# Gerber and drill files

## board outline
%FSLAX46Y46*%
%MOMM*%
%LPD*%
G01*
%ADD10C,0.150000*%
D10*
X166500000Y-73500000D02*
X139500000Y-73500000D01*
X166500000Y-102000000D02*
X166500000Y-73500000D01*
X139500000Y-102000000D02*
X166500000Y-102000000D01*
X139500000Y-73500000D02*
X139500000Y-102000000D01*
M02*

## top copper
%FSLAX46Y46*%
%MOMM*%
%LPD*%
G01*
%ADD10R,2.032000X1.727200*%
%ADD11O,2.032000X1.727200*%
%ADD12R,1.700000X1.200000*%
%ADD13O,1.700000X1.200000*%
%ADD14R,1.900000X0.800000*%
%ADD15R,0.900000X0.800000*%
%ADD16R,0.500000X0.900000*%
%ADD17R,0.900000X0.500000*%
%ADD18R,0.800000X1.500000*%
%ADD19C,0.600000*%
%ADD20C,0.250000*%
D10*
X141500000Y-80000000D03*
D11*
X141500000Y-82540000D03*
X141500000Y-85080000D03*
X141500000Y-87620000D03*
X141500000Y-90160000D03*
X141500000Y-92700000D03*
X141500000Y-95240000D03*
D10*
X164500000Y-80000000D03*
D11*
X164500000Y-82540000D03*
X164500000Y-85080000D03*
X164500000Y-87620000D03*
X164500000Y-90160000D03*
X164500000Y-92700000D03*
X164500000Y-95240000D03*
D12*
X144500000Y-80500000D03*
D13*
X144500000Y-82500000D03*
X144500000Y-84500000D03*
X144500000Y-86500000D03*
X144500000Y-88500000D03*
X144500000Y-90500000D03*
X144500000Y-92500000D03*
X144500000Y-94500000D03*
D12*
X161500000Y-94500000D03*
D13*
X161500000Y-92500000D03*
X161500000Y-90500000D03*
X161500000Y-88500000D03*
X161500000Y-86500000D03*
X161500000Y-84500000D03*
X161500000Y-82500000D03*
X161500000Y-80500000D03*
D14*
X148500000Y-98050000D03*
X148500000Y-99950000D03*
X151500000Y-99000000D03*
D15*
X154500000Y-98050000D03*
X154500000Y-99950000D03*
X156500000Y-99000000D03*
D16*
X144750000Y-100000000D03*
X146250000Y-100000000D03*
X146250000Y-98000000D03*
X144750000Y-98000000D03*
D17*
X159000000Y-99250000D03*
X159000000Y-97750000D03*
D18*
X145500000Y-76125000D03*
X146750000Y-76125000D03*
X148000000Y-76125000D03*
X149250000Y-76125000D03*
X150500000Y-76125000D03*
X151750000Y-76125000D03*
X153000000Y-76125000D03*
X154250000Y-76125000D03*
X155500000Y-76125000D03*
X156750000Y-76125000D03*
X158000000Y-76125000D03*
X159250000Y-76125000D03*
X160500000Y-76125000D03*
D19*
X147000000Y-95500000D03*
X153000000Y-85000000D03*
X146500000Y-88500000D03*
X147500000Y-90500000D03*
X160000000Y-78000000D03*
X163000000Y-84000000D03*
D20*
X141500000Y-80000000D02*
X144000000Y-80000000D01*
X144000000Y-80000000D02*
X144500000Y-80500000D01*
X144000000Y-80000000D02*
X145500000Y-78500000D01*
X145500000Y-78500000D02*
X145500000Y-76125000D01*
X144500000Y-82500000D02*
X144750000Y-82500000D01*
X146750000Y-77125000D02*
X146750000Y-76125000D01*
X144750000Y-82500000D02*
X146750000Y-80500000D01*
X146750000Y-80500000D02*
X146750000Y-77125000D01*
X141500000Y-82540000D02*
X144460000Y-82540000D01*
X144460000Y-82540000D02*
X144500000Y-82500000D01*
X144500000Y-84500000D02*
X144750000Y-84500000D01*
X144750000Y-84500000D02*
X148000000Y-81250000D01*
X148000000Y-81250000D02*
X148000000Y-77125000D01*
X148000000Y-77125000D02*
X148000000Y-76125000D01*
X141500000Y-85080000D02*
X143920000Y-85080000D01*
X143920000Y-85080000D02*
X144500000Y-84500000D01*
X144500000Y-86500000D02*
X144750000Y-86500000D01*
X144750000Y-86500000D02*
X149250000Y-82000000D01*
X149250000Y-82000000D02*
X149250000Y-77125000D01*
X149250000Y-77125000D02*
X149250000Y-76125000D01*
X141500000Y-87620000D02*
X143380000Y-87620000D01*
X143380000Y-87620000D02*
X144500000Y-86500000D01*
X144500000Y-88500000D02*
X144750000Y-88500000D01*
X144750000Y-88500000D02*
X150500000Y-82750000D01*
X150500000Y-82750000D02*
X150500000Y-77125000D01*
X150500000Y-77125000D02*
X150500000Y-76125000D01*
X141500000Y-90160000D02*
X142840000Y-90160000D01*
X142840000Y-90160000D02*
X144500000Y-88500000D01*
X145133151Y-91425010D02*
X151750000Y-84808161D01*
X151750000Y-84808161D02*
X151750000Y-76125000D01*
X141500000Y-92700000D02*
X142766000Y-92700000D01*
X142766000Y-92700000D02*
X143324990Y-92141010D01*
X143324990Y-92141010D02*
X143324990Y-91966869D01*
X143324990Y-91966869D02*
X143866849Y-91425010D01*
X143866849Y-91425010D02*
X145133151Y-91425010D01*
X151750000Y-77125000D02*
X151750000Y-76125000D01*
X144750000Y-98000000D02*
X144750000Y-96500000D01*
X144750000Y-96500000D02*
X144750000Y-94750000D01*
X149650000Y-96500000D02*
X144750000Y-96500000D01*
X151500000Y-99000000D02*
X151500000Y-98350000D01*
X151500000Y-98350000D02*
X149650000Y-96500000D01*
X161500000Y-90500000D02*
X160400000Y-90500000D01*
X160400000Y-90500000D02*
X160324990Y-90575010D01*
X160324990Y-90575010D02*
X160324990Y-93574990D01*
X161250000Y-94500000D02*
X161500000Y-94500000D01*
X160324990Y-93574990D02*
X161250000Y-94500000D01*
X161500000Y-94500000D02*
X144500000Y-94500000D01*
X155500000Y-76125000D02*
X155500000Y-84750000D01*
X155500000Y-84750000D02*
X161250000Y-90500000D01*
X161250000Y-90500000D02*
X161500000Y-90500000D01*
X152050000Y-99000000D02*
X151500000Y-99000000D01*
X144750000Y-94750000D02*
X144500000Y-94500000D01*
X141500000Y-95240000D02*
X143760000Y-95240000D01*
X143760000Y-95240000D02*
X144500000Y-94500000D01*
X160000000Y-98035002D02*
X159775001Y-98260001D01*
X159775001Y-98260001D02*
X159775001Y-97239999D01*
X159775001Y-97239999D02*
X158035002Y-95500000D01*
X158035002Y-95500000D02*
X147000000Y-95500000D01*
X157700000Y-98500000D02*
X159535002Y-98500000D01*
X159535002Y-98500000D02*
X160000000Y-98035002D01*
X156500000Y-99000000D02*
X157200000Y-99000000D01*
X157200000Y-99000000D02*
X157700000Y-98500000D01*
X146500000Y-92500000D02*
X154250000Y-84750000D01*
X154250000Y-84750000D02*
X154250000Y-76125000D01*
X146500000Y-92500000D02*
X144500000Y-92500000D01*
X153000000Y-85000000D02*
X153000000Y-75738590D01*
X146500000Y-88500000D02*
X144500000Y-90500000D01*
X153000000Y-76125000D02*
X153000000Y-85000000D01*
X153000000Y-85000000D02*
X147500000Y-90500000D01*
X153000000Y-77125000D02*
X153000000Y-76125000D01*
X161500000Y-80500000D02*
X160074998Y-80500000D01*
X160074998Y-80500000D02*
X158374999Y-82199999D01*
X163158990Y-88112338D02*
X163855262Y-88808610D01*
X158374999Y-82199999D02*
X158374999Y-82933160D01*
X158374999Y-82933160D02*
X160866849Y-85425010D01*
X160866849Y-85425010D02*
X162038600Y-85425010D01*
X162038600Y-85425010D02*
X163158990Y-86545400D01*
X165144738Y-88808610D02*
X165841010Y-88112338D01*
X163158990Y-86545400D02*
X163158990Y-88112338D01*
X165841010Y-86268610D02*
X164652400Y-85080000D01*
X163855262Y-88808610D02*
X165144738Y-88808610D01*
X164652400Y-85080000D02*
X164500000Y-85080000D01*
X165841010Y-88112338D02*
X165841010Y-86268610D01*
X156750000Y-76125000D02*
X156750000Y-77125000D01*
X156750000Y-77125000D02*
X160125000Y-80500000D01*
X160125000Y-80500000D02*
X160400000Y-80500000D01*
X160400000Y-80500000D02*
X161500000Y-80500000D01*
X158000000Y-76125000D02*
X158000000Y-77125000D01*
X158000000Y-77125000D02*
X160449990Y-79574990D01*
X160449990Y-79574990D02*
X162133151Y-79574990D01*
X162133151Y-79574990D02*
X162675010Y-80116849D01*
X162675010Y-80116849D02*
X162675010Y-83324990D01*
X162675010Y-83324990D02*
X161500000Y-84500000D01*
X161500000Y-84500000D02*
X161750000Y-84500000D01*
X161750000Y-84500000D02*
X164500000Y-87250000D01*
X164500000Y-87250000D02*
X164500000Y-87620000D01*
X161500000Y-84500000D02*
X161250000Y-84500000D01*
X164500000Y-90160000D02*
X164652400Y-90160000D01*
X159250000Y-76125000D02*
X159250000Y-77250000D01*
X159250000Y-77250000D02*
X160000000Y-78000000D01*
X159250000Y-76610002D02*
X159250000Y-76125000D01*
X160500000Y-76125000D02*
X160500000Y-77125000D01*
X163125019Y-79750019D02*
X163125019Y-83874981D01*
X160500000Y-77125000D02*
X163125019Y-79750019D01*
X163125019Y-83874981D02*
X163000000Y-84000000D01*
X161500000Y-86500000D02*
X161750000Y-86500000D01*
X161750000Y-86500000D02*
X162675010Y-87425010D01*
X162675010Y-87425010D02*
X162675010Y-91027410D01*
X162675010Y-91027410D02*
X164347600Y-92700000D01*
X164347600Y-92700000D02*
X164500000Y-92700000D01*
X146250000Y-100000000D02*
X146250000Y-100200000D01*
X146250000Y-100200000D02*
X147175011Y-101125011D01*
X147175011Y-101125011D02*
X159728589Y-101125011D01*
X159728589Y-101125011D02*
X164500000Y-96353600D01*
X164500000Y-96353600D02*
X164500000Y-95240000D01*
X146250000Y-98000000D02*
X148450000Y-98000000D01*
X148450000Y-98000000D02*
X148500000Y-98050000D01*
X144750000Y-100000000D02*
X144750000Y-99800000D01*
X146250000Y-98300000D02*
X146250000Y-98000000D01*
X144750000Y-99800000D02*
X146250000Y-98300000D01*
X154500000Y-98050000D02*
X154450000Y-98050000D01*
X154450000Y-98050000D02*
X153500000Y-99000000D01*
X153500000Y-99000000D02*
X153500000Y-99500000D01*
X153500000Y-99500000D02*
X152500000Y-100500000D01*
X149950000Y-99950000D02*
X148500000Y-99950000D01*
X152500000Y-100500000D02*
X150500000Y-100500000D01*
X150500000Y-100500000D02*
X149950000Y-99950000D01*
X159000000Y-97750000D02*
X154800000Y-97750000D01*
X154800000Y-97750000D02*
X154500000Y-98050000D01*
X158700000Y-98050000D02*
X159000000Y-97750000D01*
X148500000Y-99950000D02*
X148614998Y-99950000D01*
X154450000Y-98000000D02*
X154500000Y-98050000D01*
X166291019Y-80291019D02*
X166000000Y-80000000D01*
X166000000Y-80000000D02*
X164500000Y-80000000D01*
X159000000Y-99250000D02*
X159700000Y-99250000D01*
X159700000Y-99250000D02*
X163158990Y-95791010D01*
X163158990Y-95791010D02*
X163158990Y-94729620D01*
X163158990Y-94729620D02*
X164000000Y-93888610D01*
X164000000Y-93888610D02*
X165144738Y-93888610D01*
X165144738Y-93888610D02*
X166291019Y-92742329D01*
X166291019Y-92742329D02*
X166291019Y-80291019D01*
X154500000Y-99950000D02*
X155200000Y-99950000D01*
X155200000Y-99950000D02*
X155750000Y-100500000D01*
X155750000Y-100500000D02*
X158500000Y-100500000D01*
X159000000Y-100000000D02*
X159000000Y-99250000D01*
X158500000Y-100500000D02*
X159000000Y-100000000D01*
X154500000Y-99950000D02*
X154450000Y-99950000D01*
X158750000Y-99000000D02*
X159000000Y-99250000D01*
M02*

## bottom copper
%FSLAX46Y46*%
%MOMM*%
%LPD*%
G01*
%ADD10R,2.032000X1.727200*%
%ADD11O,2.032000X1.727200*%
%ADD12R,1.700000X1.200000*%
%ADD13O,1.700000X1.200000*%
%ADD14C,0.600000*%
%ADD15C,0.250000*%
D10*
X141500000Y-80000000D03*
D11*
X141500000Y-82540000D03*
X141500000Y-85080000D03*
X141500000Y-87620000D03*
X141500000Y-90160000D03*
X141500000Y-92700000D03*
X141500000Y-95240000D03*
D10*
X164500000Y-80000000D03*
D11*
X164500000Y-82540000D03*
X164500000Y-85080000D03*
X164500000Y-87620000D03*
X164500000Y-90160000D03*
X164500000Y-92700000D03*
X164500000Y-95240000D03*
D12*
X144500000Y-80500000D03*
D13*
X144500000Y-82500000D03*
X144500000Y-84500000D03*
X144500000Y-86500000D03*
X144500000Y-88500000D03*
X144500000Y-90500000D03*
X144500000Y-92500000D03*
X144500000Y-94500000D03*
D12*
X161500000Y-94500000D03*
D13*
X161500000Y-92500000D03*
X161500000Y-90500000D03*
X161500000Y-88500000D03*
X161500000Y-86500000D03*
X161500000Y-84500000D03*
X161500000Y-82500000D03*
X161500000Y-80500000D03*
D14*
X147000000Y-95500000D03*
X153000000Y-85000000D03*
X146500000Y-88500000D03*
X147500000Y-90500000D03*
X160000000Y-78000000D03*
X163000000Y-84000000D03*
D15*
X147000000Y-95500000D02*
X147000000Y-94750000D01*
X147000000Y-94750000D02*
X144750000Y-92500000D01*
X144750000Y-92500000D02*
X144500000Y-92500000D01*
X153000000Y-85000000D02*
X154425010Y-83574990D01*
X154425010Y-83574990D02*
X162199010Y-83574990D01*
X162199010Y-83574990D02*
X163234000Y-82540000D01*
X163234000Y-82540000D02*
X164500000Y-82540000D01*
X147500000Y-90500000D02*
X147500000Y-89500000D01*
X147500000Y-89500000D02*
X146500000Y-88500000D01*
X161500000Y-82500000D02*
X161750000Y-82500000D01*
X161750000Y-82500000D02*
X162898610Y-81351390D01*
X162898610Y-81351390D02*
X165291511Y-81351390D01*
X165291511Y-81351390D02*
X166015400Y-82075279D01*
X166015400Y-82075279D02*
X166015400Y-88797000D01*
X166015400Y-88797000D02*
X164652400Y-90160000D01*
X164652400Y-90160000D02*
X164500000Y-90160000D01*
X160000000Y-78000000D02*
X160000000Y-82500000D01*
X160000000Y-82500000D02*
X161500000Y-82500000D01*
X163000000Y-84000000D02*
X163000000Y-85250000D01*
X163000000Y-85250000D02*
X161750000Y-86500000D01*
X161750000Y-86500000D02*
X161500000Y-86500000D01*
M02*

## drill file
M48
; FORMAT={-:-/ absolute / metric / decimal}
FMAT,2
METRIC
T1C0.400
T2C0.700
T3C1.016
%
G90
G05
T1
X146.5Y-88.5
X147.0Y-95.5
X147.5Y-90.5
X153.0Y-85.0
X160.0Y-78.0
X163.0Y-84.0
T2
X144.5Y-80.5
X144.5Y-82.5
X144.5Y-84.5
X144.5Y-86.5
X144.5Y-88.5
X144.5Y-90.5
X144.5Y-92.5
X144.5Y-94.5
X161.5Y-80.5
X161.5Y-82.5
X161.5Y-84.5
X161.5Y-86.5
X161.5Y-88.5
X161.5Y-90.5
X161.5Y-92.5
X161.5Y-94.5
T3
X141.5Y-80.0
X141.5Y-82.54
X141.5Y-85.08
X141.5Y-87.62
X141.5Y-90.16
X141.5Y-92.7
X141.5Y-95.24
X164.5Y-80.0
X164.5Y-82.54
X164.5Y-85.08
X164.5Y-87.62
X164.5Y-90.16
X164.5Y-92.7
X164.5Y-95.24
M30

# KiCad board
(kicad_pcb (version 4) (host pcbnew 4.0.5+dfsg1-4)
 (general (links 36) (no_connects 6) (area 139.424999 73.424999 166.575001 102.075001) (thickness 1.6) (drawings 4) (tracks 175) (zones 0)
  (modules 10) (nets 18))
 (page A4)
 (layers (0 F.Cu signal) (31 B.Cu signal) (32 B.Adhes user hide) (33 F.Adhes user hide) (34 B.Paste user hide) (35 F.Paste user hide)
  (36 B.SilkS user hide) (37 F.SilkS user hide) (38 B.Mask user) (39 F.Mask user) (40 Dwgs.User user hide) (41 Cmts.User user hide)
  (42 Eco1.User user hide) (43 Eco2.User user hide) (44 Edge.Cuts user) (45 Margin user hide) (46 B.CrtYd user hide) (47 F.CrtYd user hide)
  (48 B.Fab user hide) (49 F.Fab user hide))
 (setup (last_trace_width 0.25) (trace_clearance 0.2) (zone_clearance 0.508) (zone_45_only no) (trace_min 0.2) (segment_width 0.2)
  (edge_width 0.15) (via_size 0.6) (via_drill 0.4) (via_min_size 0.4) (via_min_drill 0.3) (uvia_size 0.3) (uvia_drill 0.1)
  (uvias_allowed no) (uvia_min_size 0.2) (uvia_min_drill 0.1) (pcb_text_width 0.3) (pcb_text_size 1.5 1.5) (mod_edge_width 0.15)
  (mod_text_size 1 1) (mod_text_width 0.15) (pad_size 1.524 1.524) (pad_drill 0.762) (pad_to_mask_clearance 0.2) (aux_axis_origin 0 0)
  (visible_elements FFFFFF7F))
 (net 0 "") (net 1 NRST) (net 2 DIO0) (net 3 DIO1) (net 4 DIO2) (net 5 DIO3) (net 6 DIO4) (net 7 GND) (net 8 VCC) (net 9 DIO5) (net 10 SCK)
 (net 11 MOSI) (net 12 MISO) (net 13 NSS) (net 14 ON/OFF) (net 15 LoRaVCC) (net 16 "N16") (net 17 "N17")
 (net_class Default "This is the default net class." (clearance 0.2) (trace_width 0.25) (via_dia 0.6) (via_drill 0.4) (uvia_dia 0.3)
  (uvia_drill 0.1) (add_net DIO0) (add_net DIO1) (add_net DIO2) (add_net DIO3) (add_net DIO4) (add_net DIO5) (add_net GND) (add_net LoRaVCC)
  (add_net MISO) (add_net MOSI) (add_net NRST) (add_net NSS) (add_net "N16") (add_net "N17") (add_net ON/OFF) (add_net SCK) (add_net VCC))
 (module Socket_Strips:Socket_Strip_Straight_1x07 (layer F.Cu) (at 141.5 80 270)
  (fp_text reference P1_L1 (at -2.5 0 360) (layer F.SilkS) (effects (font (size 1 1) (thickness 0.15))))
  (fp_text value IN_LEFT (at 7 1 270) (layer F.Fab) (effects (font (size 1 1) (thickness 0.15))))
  (pad 1 thru_hole rect (at 0 0 270) (size 1.7272 2.032) (drill 1.016) (layers *.Cu *.Mask) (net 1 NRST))
  (pad 2 thru_hole oval (at 2.54 0 270) (size 1.7272 2.032) (drill 1.016) (layers *.Cu *.Mask) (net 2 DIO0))
  (pad 3 thru_hole oval (at 5.08 0 270) (size 1.7272 2.032) (drill 1.016) (layers *.Cu *.Mask) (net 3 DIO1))
  (pad 4 thru_hole oval (at 7.62 0 270) (size 1.7272 2.032) (drill 1.016) (layers *.Cu *.Mask) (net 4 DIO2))
  (pad 5 thru_hole oval (at 10.16 0 270) (size 1.7272 2.032) (drill 1.016) (layers *.Cu *.Mask) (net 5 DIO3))
  (pad 6 thru_hole oval (at 12.7 0 270) (size 1.7272 2.032) (drill 1.016) (layers *.Cu *.Mask) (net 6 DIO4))
  (pad 7 thru_hole oval (at 15.24 0 270) (size 1.7272 2.032) (drill 1.016) (layers *.Cu *.Mask) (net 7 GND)))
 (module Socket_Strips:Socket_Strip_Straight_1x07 (layer F.Cu) (at 164.5 80 270)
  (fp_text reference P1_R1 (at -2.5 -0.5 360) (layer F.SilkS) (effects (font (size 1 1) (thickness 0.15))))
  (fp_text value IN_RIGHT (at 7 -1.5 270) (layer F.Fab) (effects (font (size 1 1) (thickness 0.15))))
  (pad 1 thru_hole rect (at 0 0 270) (size 1.7272 2.032) (drill 1.016) (layers *.Cu *.Mask) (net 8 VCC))
  (pad 2 thru_hole oval (at 2.54 0 270) (size 1.7272 2.032) (drill 1.016) (layers *.Cu *.Mask) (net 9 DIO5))
  (pad 3 thru_hole oval (at 5.08 0 270) (size 1.7272 2.032) (drill 1.016) (layers *.Cu *.Mask) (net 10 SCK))
  (pad 4 thru_hole oval (at 7.62 0 270) (size 1.7272 2.032) (drill 1.016) (layers *.Cu *.Mask) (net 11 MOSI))
  (pad 5 thru_hole oval (at 10.16 0 270) (size 1.7272 2.032) (drill 1.016) (layers *.Cu *.Mask) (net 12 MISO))
  (pad 6 thru_hole oval (at 12.7 0 270) (size 1.7272 2.032) (drill 1.016) (layers *.Cu *.Mask) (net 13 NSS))
  (pad 7 thru_hole oval (at 15.24 0 270) (size 1.7272 2.032) (drill 1.016) (layers *.Cu *.Mask) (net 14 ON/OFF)))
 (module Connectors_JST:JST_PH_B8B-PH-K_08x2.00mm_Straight (layer F.Cu) (at 144.5 80.5 270)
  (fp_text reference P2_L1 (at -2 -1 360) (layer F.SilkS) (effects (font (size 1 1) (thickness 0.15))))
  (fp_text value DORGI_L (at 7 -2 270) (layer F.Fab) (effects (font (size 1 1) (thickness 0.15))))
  (pad 1 thru_hole rect (at 0 0 270) (size 1.2 1.7) (drill 0.7) (layers *.Cu *.Mask) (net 1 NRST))
  (pad 2 thru_hole oval (at 2 0 270) (size 1.2 1.7) (drill 0.7) (layers *.Cu *.Mask) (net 2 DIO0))
  (pad 3 thru_hole oval (at 4 0 270) (size 1.2 1.7) (drill 0.7) (layers *.Cu *.Mask) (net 3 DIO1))
  (pad 4 thru_hole oval (at 6 0 270) (size 1.2 1.7) (drill 0.7) (layers *.Cu *.Mask) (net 4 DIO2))
  (pad 5 thru_hole oval (at 8 0 270) (size 1.2 1.7) (drill 0.7) (layers *.Cu *.Mask) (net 5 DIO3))
  (pad 6 thru_hole oval (at 10 0 270) (size 1.2 1.7) (drill 0.7) (layers *.Cu *.Mask) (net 9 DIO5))
  (pad 7 thru_hole oval (at 12 0 270) (size 1.2 1.7) (drill 0.7) (layers *.Cu *.Mask) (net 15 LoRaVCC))
  (pad 8 thru_hole oval (at 14 0 270) (size 1.2 1.7) (drill 0.7) (layers *.Cu *.Mask) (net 7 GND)))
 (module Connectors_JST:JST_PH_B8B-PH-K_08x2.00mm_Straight (layer F.Cu) (at 161.5 94.5 90)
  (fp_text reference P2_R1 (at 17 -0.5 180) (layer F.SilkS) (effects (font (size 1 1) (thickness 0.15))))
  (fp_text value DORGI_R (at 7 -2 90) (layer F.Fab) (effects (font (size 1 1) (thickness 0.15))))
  (pad 1 thru_hole rect (at 0 0 90) (size 1.2 1.7) (drill 0.7) (layers *.Cu *.Mask) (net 7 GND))
  (pad 2 thru_hole oval (at 2 0 90) (size 1.2 1.7) (drill 0.7) (layers *.Cu *.Mask))
  (pad 3 thru_hole oval (at 4 0 90) (size 1.2 1.7) (drill 0.7) (layers *.Cu *.Mask) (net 7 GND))
  (pad 4 thru_hole oval (at 6 0 90) (size 1.2 1.7) (drill 0.7) (layers *.Cu *.Mask))
  (pad 5 thru_hole oval (at 8 0 90) (size 1.2 1.7) (drill 0.7) (layers *.Cu *.Mask) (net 13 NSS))
  (pad 6 thru_hole oval (at 10 0 90) (size 1.2 1.7) (drill 0.7) (layers *.Cu *.Mask) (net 11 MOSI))
  (pad 7 thru_hole oval (at 12 0 90) (size 1.2 1.7) (drill 0.7) (layers *.Cu *.Mask) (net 12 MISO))
  (pad 8 thru_hole oval (at 14 0 90) (size 1.2 1.7) (drill 0.7) (layers *.Cu *.Mask) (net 10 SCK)))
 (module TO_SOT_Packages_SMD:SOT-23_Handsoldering (layer F.Cu) (at 150 99)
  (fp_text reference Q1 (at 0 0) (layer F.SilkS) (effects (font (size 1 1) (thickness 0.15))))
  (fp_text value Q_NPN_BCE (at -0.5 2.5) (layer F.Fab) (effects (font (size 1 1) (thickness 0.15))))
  (pad 1 smd rect (at -1.5 -0.95) (size 1.9 0.8) (layers F.Cu F.Paste F.Mask) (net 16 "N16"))
  (pad 2 smd rect (at -1.5 0.95) (size 1.9 0.8) (layers F.Cu F.Paste F.Mask) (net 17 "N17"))
  (pad 3 smd rect (at 1.5 0) (size 1.9 0.8) (layers F.Cu F.Paste F.Mask) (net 7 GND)))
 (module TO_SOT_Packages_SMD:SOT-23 (layer F.Cu) (at 155.5 99)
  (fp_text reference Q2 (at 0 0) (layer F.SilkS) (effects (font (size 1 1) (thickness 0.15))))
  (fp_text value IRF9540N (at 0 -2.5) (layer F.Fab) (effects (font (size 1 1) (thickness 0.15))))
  (pad 1 smd rect (at -1 -0.95) (size 0.9 0.8) (layers F.Cu F.Paste F.Mask) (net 17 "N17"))
  (pad 2 smd rect (at -1 0.95) (size 0.9 0.8) (layers F.Cu F.Paste F.Mask) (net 8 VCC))
  (pad 3 smd rect (at 1 0) (size 0.9 0.8) (layers F.Cu F.Paste F.Mask) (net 15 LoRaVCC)))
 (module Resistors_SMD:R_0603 (layer F.Cu) (at 145.5 100)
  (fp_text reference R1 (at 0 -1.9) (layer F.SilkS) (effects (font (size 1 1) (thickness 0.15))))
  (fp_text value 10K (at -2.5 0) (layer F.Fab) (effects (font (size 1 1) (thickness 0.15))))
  (pad 1 smd rect (at -0.75 0) (size 0.5 0.9) (layers F.Cu F.Paste F.Mask) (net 16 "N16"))
  (pad 2 smd rect (at 0.75 0) (size 0.5 0.9) (layers F.Cu F.Paste F.Mask) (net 14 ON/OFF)))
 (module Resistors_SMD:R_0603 (layer F.Cu) (at 145.5 98 180)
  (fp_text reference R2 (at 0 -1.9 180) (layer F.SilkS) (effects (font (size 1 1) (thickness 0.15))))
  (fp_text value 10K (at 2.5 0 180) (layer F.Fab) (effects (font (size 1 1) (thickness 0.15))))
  (pad 1 smd rect (at -0.75 0 180) (size 0.5 0.9) (layers F.Cu F.Paste F.Mask) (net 16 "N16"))
  (pad 2 smd rect (at 0.75 0 180) (size 0.5 0.9) (layers F.Cu F.Paste F.Mask) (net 7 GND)))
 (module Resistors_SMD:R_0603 (layer F.Cu) (at 159 98.5 90)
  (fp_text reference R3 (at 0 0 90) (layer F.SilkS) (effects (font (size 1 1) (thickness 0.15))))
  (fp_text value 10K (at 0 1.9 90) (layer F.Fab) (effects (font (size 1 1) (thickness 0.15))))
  (pad 1 smd rect (at -0.75 0 90) (size 0.5 0.9) (layers F.Cu F.Paste F.Mask) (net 8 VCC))
  (pad 2 smd rect (at 0.75 0 90) (size 0.5 0.9) (layers F.Cu F.Paste F.Mask) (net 17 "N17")))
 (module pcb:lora (layer F.Cu) (at 153 77.5)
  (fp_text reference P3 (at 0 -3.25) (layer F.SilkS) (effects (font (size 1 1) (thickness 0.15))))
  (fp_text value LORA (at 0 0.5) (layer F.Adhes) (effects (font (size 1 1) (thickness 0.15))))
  (pad 1 smd rect (at -7.5 -1.375) (size 0.8 1.5) (layers F.Cu F.Paste F.Mask) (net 1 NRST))
  (pad 2 smd rect (at -6.25 -1.375) (size 0.8 1.5) (layers F.Cu F.Paste F.Mask) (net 2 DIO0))
  (pad 3 smd rect (at -5 -1.375) (size 0.8 1.5) (layers F.Cu F.Paste F.Mask) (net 3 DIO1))
  (pad 4 smd rect (at -3.75 -1.375) (size 0.8 1.5) (layers F.Cu F.Paste F.Mask) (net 4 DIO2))
  (pad 5 smd rect (at -2.5 -1.375) (size 0.8 1.5) (layers F.Cu F.Paste F.Mask) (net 5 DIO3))
  (pad 6 smd rect (at -1.25 -1.375) (size 0.8 1.5) (layers F.Cu F.Paste F.Mask) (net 6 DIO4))
  (pad 7 smd rect (at 0 -1.375) (size 0.8 1.5) (layers F.Cu F.Paste F.Mask) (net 9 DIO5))
  (pad 8 smd rect (at 1.25 -1.375) (size 0.8 1.5) (layers F.Cu F.Paste F.Mask) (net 15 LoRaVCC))
  (pad 9 smd rect (at 2.5 -1.375) (size 0.8 1.5) (layers F.Cu F.Paste F.Mask) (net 7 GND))
  (pad 10 smd rect (at 3.75 -1.375) (size 0.8 1.5) (layers F.Cu F.Paste F.Mask) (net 10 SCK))
  (pad 11 smd rect (at 5 -1.375) (size 0.8 1.5) (layers F.Cu F.Paste F.Mask) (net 11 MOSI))
  (pad 12 smd rect (at 6.25 -1.375) (size 0.8 1.5) (layers F.Cu F.Paste F.Mask) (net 12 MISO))
  (pad 13 smd rect (at 7.5 -1.375) (size 0.8 1.5) (layers F.Cu F.Paste F.Mask) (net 13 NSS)))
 (gr_line (start 166.5 73.5) (end 139.5 73.5) (layer Edge.Cuts) (width 0.15))
 (gr_line (start 166.5 102) (end 166.5 73.5) (layer Edge.Cuts) (width 0.15))
 (gr_line (start 139.5 102) (end 166.5 102) (layer Edge.Cuts) (width 0.15))
 (gr_line (start 139.5 73.5) (end 139.5 102) (layer Edge.Cuts) (width 0.15))
 (segment (start 141.5 80) (end 144 80) (width 0.25) (layer F.Cu) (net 1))
 (segment (start 144 80) (end 144.5 80.5) (width 0.25) (layer F.Cu) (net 1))
 (segment (start 144 80) (end 145.5 78.5) (width 0.25) (layer F.Cu) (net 1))
 (segment (start 145.5 78.5) (end 145.5 76.125) (width 0.25) (layer F.Cu) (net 1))
 (segment (start 144.5 82.5) (end 144.75 82.5) (width 0.25) (layer F.Cu) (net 2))
 (segment (start 146.75 77.125) (end 146.75 76.125) (width 0.25) (layer F.Cu) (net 2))
 (segment (start 144.75 82.5) (end 146.75 80.5) (width 0.25) (layer F.Cu) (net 2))
 (segment (start 146.75 80.5) (end 146.75 77.125) (width 0.25) (layer F.Cu) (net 2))
 (segment (start 141.5 82.54) (end 144.46 82.54) (width 0.25) (layer F.Cu) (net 2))
 (segment (start 144.46 82.54) (end 144.5 82.5) (width 0.25) (layer F.Cu) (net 2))
 (segment (start 144.5 84.5) (end 144.75 84.5) (width 0.25) (layer F.Cu) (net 3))
 (segment (start 144.75 84.5) (end 148 81.25) (width 0.25) (layer F.Cu) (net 3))
 (segment (start 148 81.25) (end 148 77.125) (width 0.25) (layer F.Cu) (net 3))
 (segment (start 148 77.125) (end 148 76.125) (width 0.25) (layer F.Cu) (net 3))
 (segment (start 141.5 85.08) (end 143.92 85.08) (width 0.25) (layer F.Cu) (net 3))
 (segment (start 143.92 85.08) (end 144.5 84.5) (width 0.25) (layer F.Cu) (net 3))
 (segment (start 144.5 86.5) (end 144.75 86.5) (width 0.25) (layer F.Cu) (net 4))
 (segment (start 144.75 86.5) (end 149.25 82) (width 0.25) (layer F.Cu) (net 4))
 (segment (start 149.25 82) (end 149.25 77.125) (width 0.25) (layer F.Cu) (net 4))
 (segment (start 149.25 77.125) (end 149.25 76.125) (width 0.25) (layer F.Cu) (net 4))
 (segment (start 141.5 87.62) (end 143.38 87.62) (width 0.25) (layer F.Cu) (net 4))
 (segment (start 143.38 87.62) (end 144.5 86.5) (width 0.25) (layer F.Cu) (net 4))
 (segment (start 144.5 88.5) (end 144.75 88.5) (width 0.25) (layer F.Cu) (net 5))
 (segment (start 144.75 88.5) (end 150.5 82.75) (width 0.25) (layer F.Cu) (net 5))
 (segment (start 150.5 82.75) (end 150.5 77.125) (width 0.25) (layer F.Cu) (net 5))
 (segment (start 150.5 77.125) (end 150.5 76.125) (width 0.25) (layer F.Cu) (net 5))
 (segment (start 141.5 90.16) (end 142.84 90.16) (width 0.25) (layer F.Cu) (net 5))
 (segment (start 142.84 90.16) (end 144.5 88.5) (width 0.25) (layer F.Cu) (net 5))
 (segment (start 145.133151 91.42501) (end 151.75 84.808161) (width 0.25) (layer F.Cu) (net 6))
 (segment (start 151.75 84.808161) (end 151.75 76.125) (width 0.25) (layer F.Cu) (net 6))
 (segment (start 141.5 92.7) (end 142.766 92.7) (width 0.25) (layer F.Cu) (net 6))
 (segment (start 142.766 92.7) (end 143.32499 92.14101) (width 0.25) (layer F.Cu) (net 6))
 (segment (start 143.32499 92.14101) (end 143.32499 91.966869) (width 0.25) (layer F.Cu) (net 6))
 (segment (start 143.32499 91.966869) (end 143.866849 91.42501) (width 0.25) (layer F.Cu) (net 6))
 (segment (start 143.866849 91.42501) (end 145.133151 91.42501) (width 0.25) (layer F.Cu) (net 6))
 (segment (start 151.75 77.125) (end 151.75 76.125) (width 0.25) (layer F.Cu) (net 6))
 (segment (start 144.75 98) (end 144.75 96.5) (width 0.25) (layer F.Cu) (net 7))
 (segment (start 144.75 96.5) (end 144.75 94.75) (width 0.25) (layer F.Cu) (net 7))
 (segment (start 149.65 96.5) (end 144.75 96.5) (width 0.25) (layer F.Cu) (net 7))
 (segment (start 151.5 99) (end 151.5 98.35) (width 0.25) (layer F.Cu) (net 7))
 (segment (start 151.5 98.35) (end 149.65 96.5) (width 0.25) (layer F.Cu) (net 7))
 (segment (start 161.5 90.5) (end 160.4 90.5) (width 0.25) (layer F.Cu) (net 7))
 (segment (start 160.4 90.5) (end 160.32499 90.57501) (width 0.25) (layer F.Cu) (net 7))
 (segment (start 160.32499 90.57501) (end 160.32499 93.57499) (width 0.25) (layer F.Cu) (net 7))
 (segment (start 161.25 94.5) (end 161.5 94.5) (width 0.25) (layer F.Cu) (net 7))
 (segment (start 160.32499 93.57499) (end 161.25 94.5) (width 0.25) (layer F.Cu) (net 7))
 (segment (start 161.5 94.5) (end 144.5 94.5) (width 0.25) (layer F.Cu) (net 7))
 (segment (start 155.5 76.125) (end 155.5 84.75) (width 0.25) (layer F.Cu) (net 7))
 (segment (start 155.5 84.75) (end 161.25 90.5) (width 0.25) (layer F.Cu) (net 7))
 (segment (start 161.25 90.5) (end 161.5 90.5) (width 0.25) (layer F.Cu) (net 7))
 (segment (start 152.05 99) (end 151.5 99) (width 0.25) (layer F.Cu) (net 7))
 (segment (start 144.75 94.75) (end 144.5 94.5) (width 0.25) (layer F.Cu) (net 7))
 (segment (start 141.5 95.24) (end 143.76 95.24) (width 0.25) (layer F.Cu) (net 7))
 (segment (start 143.76 95.24) (end 144.5 94.5) (width 0.25) (layer F.Cu) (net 7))
 (segment (start 147 95.5) (end 147 94.75) (width 0.25) (layer B.Cu) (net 15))
 (segment (start 147 94.75) (end 144.75 92.5) (width 0.25) (layer B.Cu) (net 15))
 (segment (start 144.75 92.5) (end 144.5 92.5) (width 0.25) (layer B.Cu) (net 15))
 (segment (start 160 98.035002) (end 159.775001 98.260001) (width 0.25) (layer F.Cu) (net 15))
 (segment (start 159.775001 98.260001) (end 159.775001 97.239999) (width 0.25) (layer F.Cu) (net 15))
 (segment (start 159.775001 97.239999) (end 158.035002 95.5) (width 0.25) (layer F.Cu) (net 15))
 (segment (start 158.035002 95.5) (end 147 95.5) (width 0.25) (layer F.Cu) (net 15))
 (via (at 147 95.5) (size 0.6) (drill 0.4) (layers F.Cu B.Cu) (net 15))
 (segment (start 157.7 98.5) (end 159.535002 98.5) (width 0.25) (layer F.Cu) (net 15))
 (segment (start 159.535002 98.5) (end 160 98.035002) (width 0.25) (layer F.Cu) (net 15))
 (segment (start 156.5 99) (end 157.2 99) (width 0.25) (layer F.Cu) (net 15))
 (segment (start 157.2 99) (end 157.7 98.5) (width 0.25) (layer F.Cu) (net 15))
 (segment (start 146.5 92.5) (end 154.25 84.75) (width 0.25) (layer F.Cu) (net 15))
 (segment (start 154.25 84.75) (end 154.25 76.125) (width 0.25) (layer F.Cu) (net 15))
 (segment (start 146.5 92.5) (end 144.5 92.5) (width 0.25) (layer F.Cu) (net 15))
 (segment (start 153 85) (end 154.42501 83.57499) (width 0.25) (layer B.Cu) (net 9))
 (segment (start 154.42501 83.57499) (end 162.19901 83.57499) (width 0.25) (layer B.Cu) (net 9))
 (segment (start 162.19901 83.57499) (end 163.234 82.54) (width 0.25) (layer B.Cu) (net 9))
 (segment (start 163.234 82.54) (end 164.5 82.54) (width 0.25) (layer B.Cu) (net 9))
 (segment (start 153 85) (end 153 75.73859) (width 0.25) (layer F.Cu) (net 9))
 (via (at 153 85) (size 0.6) (drill 0.4) (layers F.Cu B.Cu) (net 9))
 (segment (start 146.5 88.5) (end 144.5 90.5) (width 0.25) (layer F.Cu) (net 9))
 (segment (start 147.5 90.5) (end 147.5 89.5) (width 0.25) (layer B.Cu) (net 9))
 (segment (start 147.5 89.5) (end 146.5 88.5) (width 0.25) (layer B.Cu) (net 9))
 (via (at 146.5 88.5) (size 0.6) (drill 0.4) (layers F.Cu B.Cu) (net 9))
 (segment (start 153 76.125) (end 153 85) (width 0.25) (layer F.Cu) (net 9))
 (segment (start 153 85) (end 147.5 90.5) (width 0.25) (layer F.Cu) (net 9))
 (via (at 147.5 90.5) (size 0.6) (drill 0.4) (layers F.Cu B.Cu) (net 9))
 (segment (start 153 77.125) (end 153 76.125) (width 0.25) (layer F.Cu) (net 9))
 (segment (start 161.5 80.5) (end 160.074998 80.5) (width 0.25) (layer F.Cu) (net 10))
 (segment (start 160.074998 80.5) (end 158.374999 82.199999) (width 0.25) (layer F.Cu) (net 10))
 (segment (start 163.15899 88.112338) (end 163.855262 88.80861) (width 0.25) (layer F.Cu) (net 10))
 (segment (start 158.374999 82.199999) (end 158.374999 82.93316) (width 0.25) (layer F.Cu) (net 10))
 (segment (start 158.374999 82.93316) (end 160.866849 85.42501) (width 0.25) (layer F.Cu) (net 10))
 (segment (start 160.866849 85.42501) (end 162.0386 85.42501) (width 0.25) (layer F.Cu) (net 10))
 (segment (start 162.0386 85.42501) (end 163.15899 86.5454) (width 0.25) (layer F.Cu) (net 10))
 (segment (start 165.144738 88.80861) (end 165.84101 88.112338) (width 0.25) (layer F.Cu) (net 10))
 (segment (start 163.15899 86.5454) (end 163.15899 88.112338) (width 0.25) (layer F.Cu) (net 10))
 (segment (start 165.84101 86.26861) (end 164.6524 85.08) (width 0.25) (layer F.Cu) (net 10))
 (segment (start 163.855262 88.80861) (end 165.144738 88.80861) (width 0.25) (layer F.Cu) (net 10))
 (segment (start 164.6524 85.08) (end 164.5 85.08) (width 0.25) (layer F.Cu) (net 10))
 (segment (start 165.84101 88.112338) (end 165.84101 86.26861) (width 0.25) (layer F.Cu) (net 10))
 (segment (start 156.75 76.125) (end 156.75 77.125) (width 0.25) (layer F.Cu) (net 10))
 (segment (start 156.75 77.125) (end 160.125 80.5) (width 0.25) (layer F.Cu) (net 10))
 (segment (start 160.125 80.5) (end 160.4 80.5) (width 0.25) (layer F.Cu) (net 10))
 (segment (start 160.4 80.5) (end 161.5 80.5) (width 0.25) (layer F.Cu) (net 10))
 (segment (start 158 76.125) (end 158 77.125) (width 0.25) (layer F.Cu) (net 11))
 (segment (start 158 77.125) (end 160.44999 79.57499) (width 0.25) (layer F.Cu) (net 11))
 (segment (start 160.44999 79.57499) (end 162.133151 79.57499) (width 0.25) (layer F.Cu) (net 11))
 (segment (start 162.133151 79.57499) (end 162.67501 80.116849) (width 0.25) (layer F.Cu) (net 11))
 (segment (start 162.67501 80.116849) (end 162.67501 83.32499) (width 0.25) (layer F.Cu) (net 11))
 (segment (start 162.67501 83.32499) (end 161.5 84.5) (width 0.25) (layer F.Cu) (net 11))
 (segment (start 161.5 84.5) (end 161.75 84.5) (width 0.25) (layer F.Cu) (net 11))
 (segment (start 161.75 84.5) (end 164.5 87.25) (width 0.25) (layer F.Cu) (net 11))
 (segment (start 164.5 87.25) (end 164.5 87.62) (width 0.25) (layer F.Cu) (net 11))
 (segment (start 161.5 84.5) (end 161.25 84.5) (width 0.25) (layer F.Cu) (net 11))
 (segment (start 161.5 82.5) (end 161.75 82.5) (width 0.25) (layer B.Cu) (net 12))
 (segment (start 161.75 82.5) (end 162.89861 81.35139) (width 0.25) (layer B.Cu) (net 12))
 (segment (start 162.89861 81.35139) (end 165.291511 81.35139) (width 0.25) (layer B.Cu) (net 12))
 (segment (start 165.291511 81.35139) (end 166.0154 82.075279) (width 0.25) (layer B.Cu) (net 12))
 (segment (start 166.0154 82.075279) (end 166.0154 88.797) (width 0.25) (layer B.Cu) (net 12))
 (segment (start 166.0154 88.797) (end 164.6524 90.16) (width 0.25) (layer B.Cu) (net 12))
 (segment (start 164.6524 90.16) (end 164.5 90.16) (width 0.25) (layer B.Cu) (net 12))
 (segment (start 160 78) (end 160 82.5) (width 0.25) (layer B.Cu) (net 12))
 (segment (start 160 82.5) (end 161.5 82.5) (width 0.25) (layer B.Cu) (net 12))
 (segment (start 164.5 90.16) (end 164.6524 90.16) (width 0.25) (layer F.Cu) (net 12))
 (segment (start 159.25 76.125) (end 159.25 77.25) (width 0.25) (layer F.Cu) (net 12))
 (segment (start 159.25 77.25) (end 160 78) (width 0.25) (layer F.Cu) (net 12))
 (via (at 160 78) (size 0.6) (drill 0.4) (layers F.Cu B.Cu) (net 12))
 (segment (start 159.25 76.610002) (end 159.25 76.125) (width 0.25) (layer F.Cu) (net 12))
 (segment (start 163 84) (end 163 85.25) (width 0.25) (layer B.Cu) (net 13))
 (segment (start 163 85.25) (end 161.75 86.5) (width 0.25) (layer B.Cu) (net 13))
 (segment (start 161.75 86.5) (end 161.5 86.5) (width 0.25) (layer B.Cu) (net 13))
 (segment (start 160.5 76.125) (end 160.5 77.125) (width 0.25) (layer F.Cu) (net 13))
 (segment (start 163.125019 79.750019) (end 163.125019 83.874981) (width 0.25) (layer F.Cu) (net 13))
 (segment (start 160.5 77.125) (end 163.125019 79.750019) (width 0.25) (layer F.Cu) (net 13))
 (segment (start 163.125019 83.874981) (end 163 84) (width 0.25) (layer F.Cu) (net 13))
 (via (at 163 84) (size 0.6) (drill 0.4) (layers F.Cu B.Cu) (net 13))
 (segment (start 161.5 86.5) (end 161.75 86.5) (width 0.25) (layer F.Cu) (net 13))
 (segment (start 161.75 86.5) (end 162.67501 87.42501) (width 0.25) (layer F.Cu) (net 13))
 (segment (start 162.67501 87.42501) (end 162.67501 91.02741) (width 0.25) (layer F.Cu) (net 13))
 (segment (start 162.67501 91.02741) (end 164.3476 92.7) (width 0.25) (layer F.Cu) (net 13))
 (segment (start 164.3476 92.7) (end 164.5 92.7) (width 0.25) (layer F.Cu) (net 13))
 (segment (start 146.25 100) (end 146.25 100.2) (width 0.25) (layer F.Cu) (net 14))
 (segment (start 146.25 100.2) (end 147.175011 101.125011) (width 0.25) (layer F.Cu) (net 14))
 (segment (start 147.175011 101.125011) (end 159.728589 101.125011) (width 0.25) (layer F.Cu) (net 14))
 (segment (start 159.728589 101.125011) (end 164.5 96.3536) (width 0.25) (layer F.Cu) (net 14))
 (segment (start 164.5 96.3536) (end 164.5 95.24) (width 0.25) (layer F.Cu) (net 14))
 (segment (start 146.25 98) (end 148.45 98) (width 0.25) (layer F.Cu) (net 16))
 (segment (start 148.45 98) (end 148.5 98.05) (width 0.25) (layer F.Cu) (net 16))
 (segment (start 144.75 100) (end 144.75 99.8) (width 0.25) (layer F.Cu) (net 16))
 (segment (start 146.25 98.3) (end 146.25 98) (width 0.25) (layer F.Cu) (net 16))
 (segment (start 144.75 99.8) (end 146.25 98.3) (width 0.25) (layer F.Cu) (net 16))
 (segment (start 154.5 98.05) (end 154.45 98.05) (width 0.25) (layer F.Cu) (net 17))
 (segment (start 154.45 98.05) (end 153.5 99) (width 0.25) (layer F.Cu) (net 17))
 (segment (start 153.5 99) (end 153.5 99.5) (width 0.25) (layer F.Cu) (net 17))
 (segment (start 153.5 99.5) (end 152.5 100.5) (width 0.25) (layer F.Cu) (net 17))
 (segment (start 149.95 99.95) (end 148.5 99.95) (width 0.25) (layer F.Cu) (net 17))
 (segment (start 152.5 100.5) (end 150.5 100.5) (width 0.25) (layer F.Cu) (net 17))
 (segment (start 150.5 100.5) (end 149.95 99.95) (width 0.25) (layer F.Cu) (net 17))
 (segment (start 159 97.75) (end 154.8 97.75) (width 0.25) (layer F.Cu) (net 17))
 (segment (start 154.8 97.75) (end 154.5 98.05) (width 0.25) (layer F.Cu) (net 17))
 (segment (start 158.7 98.05) (end 159 97.75) (width 0.25) (layer F.Cu) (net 17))
 (segment (start 148.5 99.95) (end 148.614998 99.95) (width 0.25) (layer F.Cu) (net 17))
 (segment (start 154.45 98) (end 154.5 98.05) (width 0.25) (layer F.Cu) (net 17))
 (segment (start 166.291019 80.291019) (end 166 80) (width 0.25) (layer F.Cu) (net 8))
 (segment (start 166 80) (end 164.5 80) (width 0.25) (layer F.Cu) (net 8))
 (segment (start 159 99.25) (end 159.7 99.25) (width 0.25) (layer F.Cu) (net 8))
 (segment (start 159.7 99.25) (end 163.15899 95.79101) (width 0.25) (layer F.Cu) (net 8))
 (segment (start 163.15899 95.79101) (end 163.15899 94.72962) (width 0.25) (layer F.Cu) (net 8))
 (segment (start 163.15899 94.72962) (end 164 93.88861) (width 0.25) (layer F.Cu) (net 8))
 (segment (start 164 93.88861) (end 165.144738 93.88861) (width 0.25) (layer F.Cu) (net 8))
 (segment (start 165.144738 93.88861) (end 166.291019 92.742329) (width 0.25) (layer F.Cu) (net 8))
 (segment (start 166.291019 92.742329) (end 166.291019 80.291019) (width 0.25) (layer F.Cu) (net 8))
 (segment (start 154.5 99.95) (end 155.2 99.95) (width 0.25) (layer F.Cu) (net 8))
 (segment (start 155.2 99.95) (end 155.75 100.5) (width 0.25) (layer F.Cu) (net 8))
 (segment (start 155.75 100.5) (end 158.5 100.5) (width 0.25) (layer F.Cu) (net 8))
 (segment (start 159 100) (end 159 99.25) (width 0.25) (layer F.Cu) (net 8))
 (segment (start 158.5 100.5) (end 159 100) (width 0.25) (layer F.Cu) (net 8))
 (segment (start 154.5 99.95) (end 154.45 99.95) (width 0.25) (layer F.Cu) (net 8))
 (segment (start 158.75 99) (end 159 99.25) (width 0.25) (layer F.Cu) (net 8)))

